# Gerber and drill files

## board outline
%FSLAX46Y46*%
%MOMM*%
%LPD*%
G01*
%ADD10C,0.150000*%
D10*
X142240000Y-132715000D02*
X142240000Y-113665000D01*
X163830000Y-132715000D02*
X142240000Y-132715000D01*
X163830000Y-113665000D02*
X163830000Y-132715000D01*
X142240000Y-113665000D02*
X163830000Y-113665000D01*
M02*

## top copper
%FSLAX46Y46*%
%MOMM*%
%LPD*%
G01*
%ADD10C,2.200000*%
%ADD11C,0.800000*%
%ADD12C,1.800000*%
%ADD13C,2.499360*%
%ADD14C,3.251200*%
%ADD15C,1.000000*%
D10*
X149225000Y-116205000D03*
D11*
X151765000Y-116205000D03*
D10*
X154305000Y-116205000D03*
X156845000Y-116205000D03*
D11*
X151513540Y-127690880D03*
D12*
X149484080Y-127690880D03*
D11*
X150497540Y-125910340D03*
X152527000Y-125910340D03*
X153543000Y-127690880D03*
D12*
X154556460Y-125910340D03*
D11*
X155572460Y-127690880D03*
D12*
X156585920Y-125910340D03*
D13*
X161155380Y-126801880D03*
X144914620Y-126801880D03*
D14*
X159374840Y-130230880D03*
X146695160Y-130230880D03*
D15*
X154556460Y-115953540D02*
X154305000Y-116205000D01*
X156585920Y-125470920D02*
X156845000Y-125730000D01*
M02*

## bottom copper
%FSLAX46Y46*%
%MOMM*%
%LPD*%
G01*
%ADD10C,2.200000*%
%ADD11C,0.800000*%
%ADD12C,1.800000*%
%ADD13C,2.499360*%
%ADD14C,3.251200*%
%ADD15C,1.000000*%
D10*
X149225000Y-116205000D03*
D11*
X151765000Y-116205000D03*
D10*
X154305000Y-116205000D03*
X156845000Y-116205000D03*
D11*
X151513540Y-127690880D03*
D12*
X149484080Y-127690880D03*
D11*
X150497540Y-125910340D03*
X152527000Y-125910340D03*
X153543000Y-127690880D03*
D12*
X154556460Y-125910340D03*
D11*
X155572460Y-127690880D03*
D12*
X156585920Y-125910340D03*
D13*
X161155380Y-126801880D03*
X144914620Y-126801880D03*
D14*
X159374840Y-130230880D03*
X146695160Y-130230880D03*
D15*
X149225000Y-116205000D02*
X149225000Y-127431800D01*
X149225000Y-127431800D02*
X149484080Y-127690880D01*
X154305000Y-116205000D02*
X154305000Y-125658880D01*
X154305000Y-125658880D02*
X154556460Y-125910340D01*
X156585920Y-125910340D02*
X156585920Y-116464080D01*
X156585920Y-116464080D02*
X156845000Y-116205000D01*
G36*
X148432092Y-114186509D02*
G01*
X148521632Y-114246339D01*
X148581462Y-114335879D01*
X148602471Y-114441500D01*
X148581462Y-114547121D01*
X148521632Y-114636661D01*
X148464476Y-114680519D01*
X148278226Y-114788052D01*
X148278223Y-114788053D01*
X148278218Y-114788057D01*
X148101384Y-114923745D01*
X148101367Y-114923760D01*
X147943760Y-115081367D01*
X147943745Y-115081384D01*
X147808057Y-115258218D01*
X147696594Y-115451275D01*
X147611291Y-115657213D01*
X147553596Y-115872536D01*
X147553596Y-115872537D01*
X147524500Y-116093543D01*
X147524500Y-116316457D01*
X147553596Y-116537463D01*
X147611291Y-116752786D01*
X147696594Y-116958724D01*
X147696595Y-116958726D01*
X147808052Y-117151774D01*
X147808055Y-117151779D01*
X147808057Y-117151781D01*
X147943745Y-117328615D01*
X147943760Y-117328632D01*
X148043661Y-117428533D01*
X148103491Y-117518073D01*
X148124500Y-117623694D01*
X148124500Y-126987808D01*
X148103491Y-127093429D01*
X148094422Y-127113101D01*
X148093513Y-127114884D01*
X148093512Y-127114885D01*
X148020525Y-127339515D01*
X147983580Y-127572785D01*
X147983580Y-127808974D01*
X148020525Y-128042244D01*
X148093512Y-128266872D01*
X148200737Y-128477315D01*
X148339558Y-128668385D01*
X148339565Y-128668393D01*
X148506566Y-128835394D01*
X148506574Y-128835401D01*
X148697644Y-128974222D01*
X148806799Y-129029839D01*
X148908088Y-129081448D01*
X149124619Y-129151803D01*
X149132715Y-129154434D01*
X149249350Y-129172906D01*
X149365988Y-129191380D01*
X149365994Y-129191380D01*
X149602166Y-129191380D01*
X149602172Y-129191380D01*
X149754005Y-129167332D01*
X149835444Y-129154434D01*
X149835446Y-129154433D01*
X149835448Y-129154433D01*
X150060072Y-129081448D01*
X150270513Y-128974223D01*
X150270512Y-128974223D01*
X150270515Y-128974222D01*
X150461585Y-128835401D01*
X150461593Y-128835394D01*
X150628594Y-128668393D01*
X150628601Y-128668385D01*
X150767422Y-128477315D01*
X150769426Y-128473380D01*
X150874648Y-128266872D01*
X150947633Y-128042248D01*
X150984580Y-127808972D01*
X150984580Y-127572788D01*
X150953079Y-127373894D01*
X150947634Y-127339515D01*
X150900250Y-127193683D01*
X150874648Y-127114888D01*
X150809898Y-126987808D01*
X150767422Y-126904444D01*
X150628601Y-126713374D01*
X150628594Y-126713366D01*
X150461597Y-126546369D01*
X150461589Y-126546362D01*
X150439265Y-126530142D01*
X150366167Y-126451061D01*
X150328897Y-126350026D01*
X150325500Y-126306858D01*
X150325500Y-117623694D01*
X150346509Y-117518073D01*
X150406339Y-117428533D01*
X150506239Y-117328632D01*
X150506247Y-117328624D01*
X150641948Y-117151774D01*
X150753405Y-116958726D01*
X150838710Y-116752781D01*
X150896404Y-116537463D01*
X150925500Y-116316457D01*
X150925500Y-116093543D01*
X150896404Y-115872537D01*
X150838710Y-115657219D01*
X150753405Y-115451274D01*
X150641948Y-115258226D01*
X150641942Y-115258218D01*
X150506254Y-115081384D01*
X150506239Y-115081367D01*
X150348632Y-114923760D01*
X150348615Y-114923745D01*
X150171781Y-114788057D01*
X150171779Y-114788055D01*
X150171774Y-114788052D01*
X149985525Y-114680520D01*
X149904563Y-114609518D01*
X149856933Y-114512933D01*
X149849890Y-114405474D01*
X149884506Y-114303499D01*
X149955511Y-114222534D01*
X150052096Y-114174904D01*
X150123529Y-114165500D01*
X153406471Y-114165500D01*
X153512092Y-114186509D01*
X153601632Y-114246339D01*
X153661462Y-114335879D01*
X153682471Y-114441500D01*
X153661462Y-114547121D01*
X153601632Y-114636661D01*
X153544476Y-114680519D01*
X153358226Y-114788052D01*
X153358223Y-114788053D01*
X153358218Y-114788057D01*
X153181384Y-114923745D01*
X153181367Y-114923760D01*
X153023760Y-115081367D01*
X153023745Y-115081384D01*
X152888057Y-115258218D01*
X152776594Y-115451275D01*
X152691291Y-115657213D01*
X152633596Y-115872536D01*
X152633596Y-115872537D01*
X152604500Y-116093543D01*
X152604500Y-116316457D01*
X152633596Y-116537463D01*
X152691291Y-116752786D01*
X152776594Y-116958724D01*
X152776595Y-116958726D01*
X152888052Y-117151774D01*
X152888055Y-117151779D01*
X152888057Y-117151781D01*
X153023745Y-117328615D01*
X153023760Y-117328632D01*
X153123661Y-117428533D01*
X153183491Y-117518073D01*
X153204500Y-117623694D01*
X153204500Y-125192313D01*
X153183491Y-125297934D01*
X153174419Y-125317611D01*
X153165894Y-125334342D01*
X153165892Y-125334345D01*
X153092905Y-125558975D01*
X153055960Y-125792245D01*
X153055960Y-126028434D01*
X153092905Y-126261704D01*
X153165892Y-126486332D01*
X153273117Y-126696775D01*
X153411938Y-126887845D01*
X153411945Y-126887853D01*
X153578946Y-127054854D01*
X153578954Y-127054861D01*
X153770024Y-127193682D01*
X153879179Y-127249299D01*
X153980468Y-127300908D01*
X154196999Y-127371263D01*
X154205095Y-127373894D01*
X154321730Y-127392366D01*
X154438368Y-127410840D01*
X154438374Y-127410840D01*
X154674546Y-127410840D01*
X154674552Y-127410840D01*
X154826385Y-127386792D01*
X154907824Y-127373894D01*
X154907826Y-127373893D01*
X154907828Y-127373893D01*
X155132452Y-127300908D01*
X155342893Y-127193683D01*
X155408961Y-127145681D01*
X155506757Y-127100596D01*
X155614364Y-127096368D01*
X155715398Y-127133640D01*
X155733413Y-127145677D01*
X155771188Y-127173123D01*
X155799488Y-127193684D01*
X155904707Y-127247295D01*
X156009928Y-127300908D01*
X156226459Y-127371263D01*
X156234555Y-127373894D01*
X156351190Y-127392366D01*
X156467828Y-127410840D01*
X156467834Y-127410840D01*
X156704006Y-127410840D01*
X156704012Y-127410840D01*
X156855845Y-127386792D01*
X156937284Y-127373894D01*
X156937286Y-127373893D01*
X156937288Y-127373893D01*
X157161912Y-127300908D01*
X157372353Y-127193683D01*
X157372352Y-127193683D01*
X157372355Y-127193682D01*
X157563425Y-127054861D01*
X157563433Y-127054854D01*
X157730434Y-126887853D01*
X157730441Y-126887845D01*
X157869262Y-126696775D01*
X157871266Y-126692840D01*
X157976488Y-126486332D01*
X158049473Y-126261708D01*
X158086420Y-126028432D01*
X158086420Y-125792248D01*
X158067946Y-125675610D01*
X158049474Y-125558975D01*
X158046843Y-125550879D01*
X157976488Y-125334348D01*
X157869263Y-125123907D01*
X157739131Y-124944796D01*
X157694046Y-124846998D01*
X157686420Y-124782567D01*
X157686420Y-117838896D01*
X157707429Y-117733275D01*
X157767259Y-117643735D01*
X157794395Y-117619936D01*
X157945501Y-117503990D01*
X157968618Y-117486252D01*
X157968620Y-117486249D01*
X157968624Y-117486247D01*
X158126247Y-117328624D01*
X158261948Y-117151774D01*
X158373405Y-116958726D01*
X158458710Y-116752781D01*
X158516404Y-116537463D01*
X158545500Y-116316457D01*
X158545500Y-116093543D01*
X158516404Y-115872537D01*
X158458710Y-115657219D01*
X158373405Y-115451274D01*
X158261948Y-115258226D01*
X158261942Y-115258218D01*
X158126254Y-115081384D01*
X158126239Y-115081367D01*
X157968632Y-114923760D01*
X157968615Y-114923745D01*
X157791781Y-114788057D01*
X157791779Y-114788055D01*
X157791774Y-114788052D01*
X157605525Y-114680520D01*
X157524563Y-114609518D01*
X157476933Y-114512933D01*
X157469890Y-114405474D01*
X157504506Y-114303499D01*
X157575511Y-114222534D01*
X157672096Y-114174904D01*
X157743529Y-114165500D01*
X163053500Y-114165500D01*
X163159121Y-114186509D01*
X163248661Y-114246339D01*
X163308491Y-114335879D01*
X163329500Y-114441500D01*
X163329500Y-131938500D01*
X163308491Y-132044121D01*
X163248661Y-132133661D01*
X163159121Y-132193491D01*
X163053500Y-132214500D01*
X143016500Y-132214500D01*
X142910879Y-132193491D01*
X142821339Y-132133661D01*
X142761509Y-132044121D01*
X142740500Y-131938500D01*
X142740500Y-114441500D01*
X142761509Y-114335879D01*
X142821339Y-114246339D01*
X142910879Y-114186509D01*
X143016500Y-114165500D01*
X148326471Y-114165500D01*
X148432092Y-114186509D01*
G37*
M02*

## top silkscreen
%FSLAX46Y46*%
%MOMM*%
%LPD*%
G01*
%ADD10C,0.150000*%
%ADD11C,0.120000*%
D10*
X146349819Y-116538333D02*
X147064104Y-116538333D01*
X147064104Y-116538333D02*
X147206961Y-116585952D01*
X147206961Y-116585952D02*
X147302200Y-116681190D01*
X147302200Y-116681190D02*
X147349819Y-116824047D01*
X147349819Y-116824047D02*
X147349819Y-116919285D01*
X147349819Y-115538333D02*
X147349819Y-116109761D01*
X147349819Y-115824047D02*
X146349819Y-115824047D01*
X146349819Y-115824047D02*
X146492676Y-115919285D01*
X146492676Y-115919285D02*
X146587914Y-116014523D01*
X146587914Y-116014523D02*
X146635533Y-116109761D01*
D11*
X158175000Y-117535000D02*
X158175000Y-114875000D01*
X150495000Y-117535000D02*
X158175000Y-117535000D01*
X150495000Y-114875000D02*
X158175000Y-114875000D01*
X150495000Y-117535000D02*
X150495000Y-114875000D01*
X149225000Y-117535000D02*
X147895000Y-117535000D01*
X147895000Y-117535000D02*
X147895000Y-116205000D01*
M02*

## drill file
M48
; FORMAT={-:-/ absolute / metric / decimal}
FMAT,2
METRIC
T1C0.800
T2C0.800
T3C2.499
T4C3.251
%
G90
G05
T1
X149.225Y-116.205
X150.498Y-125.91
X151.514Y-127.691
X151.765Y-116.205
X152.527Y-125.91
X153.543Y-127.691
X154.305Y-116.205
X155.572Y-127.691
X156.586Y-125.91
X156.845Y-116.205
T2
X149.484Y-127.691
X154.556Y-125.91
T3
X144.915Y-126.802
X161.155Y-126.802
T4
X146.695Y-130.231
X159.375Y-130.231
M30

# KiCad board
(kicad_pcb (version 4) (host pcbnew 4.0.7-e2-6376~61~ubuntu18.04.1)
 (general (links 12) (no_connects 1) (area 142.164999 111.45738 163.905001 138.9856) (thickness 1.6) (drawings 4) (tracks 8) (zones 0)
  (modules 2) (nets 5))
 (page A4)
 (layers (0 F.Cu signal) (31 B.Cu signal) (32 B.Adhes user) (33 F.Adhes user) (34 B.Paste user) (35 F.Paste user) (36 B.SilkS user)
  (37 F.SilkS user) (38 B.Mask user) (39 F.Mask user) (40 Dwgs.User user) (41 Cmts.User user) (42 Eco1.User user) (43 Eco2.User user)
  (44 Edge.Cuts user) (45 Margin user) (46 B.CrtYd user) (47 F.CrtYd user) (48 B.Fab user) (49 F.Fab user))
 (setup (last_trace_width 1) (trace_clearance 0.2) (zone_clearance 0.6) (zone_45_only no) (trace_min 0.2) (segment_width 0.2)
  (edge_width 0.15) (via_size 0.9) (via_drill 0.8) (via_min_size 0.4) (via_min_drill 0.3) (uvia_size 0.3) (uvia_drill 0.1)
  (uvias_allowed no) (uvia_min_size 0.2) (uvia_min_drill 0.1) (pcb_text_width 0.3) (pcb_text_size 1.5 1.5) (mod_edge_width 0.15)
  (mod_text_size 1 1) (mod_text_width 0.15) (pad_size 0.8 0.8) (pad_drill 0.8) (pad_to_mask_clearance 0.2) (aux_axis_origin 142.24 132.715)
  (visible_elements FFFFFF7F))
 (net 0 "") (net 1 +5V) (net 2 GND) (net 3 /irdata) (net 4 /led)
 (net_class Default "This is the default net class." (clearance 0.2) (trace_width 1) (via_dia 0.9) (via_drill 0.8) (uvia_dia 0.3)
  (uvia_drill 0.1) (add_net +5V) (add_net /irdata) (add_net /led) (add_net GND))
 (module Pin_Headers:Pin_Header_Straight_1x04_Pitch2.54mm (layer F.Cu) (at 149.225 116.205 90)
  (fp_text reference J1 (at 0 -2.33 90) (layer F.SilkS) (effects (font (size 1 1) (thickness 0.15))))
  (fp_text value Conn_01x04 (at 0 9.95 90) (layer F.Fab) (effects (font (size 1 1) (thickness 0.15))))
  (fp_line (start -1.33 8.95) (end 1.33 8.95) (layer F.SilkS) (width 0.12))
  (fp_line (start -1.33 1.27) (end -1.33 8.95) (layer F.SilkS) (width 0.12))
  (fp_line (start 1.33 1.27) (end 1.33 8.95) (layer F.SilkS) (width 0.12))
  (fp_line (start -1.33 1.27) (end 1.33 1.27) (layer F.SilkS) (width 0.12))
  (fp_line (start -1.33 0) (end -1.33 -1.33) (layer F.SilkS) (width 0.12))
  (fp_line (start -1.33 -1.33) (end 0 -1.33) (layer F.SilkS) (width 0.12))
  (pad 1 thru_hole circle (at 0 0 90) (size 2.2 2.2) (drill 0.8) (layers *.Cu *.Mask) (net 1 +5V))
  (pad 2 thru_hole circle (at 0 2.54 90) (size 0.8 0.8) (drill 0.8) (layers *.Cu *.Mask) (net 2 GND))
  (pad 3 thru_hole circle (at 0 5.08 90) (size 2.2 2.2) (drill 0.8) (layers *.Cu *.Mask) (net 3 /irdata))
  (pad 4 thru_hole circle (at 0 7.62 90) (size 2.2 2.2) (drill 0.8) (layers *.Cu *.Mask) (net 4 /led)))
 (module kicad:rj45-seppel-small (layer B.Cu) (at 153.035 127.635 180)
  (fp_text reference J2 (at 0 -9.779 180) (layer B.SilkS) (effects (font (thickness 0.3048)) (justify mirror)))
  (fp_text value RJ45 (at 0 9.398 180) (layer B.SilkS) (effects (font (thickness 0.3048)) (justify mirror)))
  (pad 3 thru_hole circle (at 1.52146 -0.05588 180) (size 0.8 0.8) (drill 0.8) (layers *.Cu *.Mask) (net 2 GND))
  (pad 1 thru_hole circle (at 3.55092 -0.05588 180) (size 1.8 1.8) (drill 0.8001) (layers *.Cu *.Mask) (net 1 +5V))
  (pad 2 thru_hole circle (at 2.53746 1.72466 180) (size 0.8 0.8) (drill 0.8) (layers *.Cu *.Mask) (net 2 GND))
  (pad 4 thru_hole circle (at 0.508 1.72466 180) (size 0.8 0.8) (drill 0.8) (layers *.Cu *.Mask) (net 2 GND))
  (pad 5 thru_hole circle (at -0.508 -0.05588 180) (size 0.8 0.8) (drill 0.8) (layers *.Cu *.Mask) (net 2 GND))
  (pad 6 thru_hole circle (at -1.52146 1.72466 180) (size 1.8 1.8) (drill 0.8001) (layers *.Cu *.Mask) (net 3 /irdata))
  (pad 7 thru_hole circle (at -2.53746 -0.05588 180) (size 0.8 0.8) (drill 0.8) (layers *.Cu *.Mask) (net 2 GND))
  (pad 8 thru_hole circle (at -3.55092 1.72466 180) (size 1.8 1.8) (drill 0.8) (layers *.Cu *.Mask) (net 4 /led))
  (pad 13 thru_hole circle (at -8.12038 0.83312 180) (size 2.49936 2.49936) (drill 2.49936) (layers *.Cu *.Mask) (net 2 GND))
  (pad 13 thru_hole circle (at 8.12038 0.83312 180) (size 2.49936 2.49936) (drill 2.49936) (layers *.Cu *.Mask) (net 2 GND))
  (pad "" thru_hole circle (at -6.33984 -2.59588 180) (size 3.2512 3.2512) (drill 3.2512) (layers *.Cu *.Mask) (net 2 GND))
  (pad "" thru_hole circle (at 6.33984 -2.59588 180) (size 3.2512 3.2512) (drill 3.2512) (layers *.Cu *.Mask) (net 2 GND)))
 (gr_line (start 142.24 132.715) (end 142.24 113.665) (angle 90) (layer Edge.Cuts) (width 0.15))
 (gr_line (start 163.83 132.715) (end 142.24 132.715) (angle 90) (layer Edge.Cuts) (width 0.15))
 (gr_line (start 163.83 113.665) (end 163.83 132.715) (angle 90) (layer Edge.Cuts) (width 0.15))
 (gr_line (start 142.24 113.665) (end 163.83 113.665) (angle 90) (layer Edge.Cuts) (width 0.15))
 (segment (start 149.225 116.205) (end 149.225 127.4318) (width 1) (layer B.Cu) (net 1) (status C00000))
 (segment (start 149.225 127.4318) (end 149.48408 127.69088) (width 1) (layer B.Cu) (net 1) (status C00000))
 (segment (start 154.305 116.205) (end 154.305 125.65888) (width 1) (layer B.Cu) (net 3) (status C00000))
 (segment (start 154.305 125.65888) (end 154.55646 125.91034) (width 1) (layer B.Cu) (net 3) (status C00000))
 (segment (start 154.55646 115.95354) (end 154.305 116.205) (width 1) (layer F.Cu) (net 3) (status 30))
 (segment (start 156.58592 125.91034) (end 156.58592 116.46408) (width 1) (layer B.Cu) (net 4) (status C00000))
 (segment (start 156.58592 116.46408) (end 156.845 116.205) (width 1) (layer B.Cu) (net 4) (status C00000))
 (segment (start 156.58592 125.47092) (end 156.845 125.73) (width 1) (layer F.Cu) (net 4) (status 30))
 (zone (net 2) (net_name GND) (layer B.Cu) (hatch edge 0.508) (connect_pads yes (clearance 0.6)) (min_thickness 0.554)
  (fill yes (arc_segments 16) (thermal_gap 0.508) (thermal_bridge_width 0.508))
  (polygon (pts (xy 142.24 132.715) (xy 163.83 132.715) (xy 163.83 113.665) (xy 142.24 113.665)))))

